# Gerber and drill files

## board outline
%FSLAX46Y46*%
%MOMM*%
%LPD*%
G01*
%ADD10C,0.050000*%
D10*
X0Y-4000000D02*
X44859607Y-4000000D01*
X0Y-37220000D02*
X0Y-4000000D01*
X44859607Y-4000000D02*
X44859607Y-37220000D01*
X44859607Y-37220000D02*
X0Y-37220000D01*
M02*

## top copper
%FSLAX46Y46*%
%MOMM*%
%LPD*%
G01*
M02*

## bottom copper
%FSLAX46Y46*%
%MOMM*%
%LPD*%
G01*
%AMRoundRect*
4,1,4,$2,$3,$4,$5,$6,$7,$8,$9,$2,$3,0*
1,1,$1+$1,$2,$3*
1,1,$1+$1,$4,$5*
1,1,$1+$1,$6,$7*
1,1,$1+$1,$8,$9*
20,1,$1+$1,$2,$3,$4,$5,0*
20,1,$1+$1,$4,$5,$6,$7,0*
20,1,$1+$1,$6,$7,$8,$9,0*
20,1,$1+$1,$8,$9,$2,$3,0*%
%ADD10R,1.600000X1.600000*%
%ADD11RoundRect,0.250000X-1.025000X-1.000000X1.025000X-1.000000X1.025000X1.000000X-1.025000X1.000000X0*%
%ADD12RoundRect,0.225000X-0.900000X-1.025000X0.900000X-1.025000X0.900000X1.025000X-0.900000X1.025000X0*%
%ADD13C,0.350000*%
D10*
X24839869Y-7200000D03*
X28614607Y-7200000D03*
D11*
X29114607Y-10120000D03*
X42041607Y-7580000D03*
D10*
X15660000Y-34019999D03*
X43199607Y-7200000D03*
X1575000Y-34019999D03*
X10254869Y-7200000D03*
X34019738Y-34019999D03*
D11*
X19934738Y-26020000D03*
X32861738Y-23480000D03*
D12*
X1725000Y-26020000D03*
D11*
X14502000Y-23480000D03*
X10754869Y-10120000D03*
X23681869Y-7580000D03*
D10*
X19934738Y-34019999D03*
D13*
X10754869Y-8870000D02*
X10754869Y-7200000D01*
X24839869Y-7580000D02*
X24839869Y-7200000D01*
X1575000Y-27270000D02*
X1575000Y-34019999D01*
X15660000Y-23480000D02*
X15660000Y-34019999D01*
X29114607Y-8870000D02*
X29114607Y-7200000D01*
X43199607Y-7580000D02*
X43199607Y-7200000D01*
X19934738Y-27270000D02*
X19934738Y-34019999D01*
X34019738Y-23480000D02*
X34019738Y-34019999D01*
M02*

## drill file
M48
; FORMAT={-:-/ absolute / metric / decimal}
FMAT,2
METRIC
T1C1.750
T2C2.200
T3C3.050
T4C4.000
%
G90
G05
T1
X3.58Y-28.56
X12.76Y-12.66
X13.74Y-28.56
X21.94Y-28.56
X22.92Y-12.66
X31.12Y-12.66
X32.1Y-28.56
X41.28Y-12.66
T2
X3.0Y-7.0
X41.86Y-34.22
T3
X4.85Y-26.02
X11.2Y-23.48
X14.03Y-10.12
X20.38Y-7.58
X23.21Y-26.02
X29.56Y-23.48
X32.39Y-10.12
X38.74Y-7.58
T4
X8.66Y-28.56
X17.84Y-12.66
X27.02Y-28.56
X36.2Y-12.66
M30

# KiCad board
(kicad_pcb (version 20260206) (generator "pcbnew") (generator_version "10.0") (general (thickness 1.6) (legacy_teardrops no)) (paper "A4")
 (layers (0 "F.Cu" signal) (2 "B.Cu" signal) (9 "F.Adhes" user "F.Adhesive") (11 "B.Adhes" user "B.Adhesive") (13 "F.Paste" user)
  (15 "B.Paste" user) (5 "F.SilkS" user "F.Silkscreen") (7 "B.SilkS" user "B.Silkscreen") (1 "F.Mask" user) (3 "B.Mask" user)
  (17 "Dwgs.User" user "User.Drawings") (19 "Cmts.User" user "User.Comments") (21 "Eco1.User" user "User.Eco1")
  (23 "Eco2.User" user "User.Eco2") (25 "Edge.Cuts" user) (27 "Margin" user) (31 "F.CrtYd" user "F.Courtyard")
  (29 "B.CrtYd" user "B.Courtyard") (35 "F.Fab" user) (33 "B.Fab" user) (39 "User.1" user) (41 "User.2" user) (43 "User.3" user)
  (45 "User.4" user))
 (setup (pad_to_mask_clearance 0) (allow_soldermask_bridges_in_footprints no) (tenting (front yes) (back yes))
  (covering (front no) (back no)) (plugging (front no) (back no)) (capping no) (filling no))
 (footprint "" (layer "F.Cu") (at 0 0)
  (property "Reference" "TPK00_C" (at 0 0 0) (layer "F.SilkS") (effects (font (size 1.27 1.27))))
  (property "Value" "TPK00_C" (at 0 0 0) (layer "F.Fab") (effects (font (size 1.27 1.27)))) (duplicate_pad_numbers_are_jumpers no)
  (pad "1" smd rect (at 24.839869 7.2) (size 1.6 1.6) (layers "B.Cu" "B.Mask") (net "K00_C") (thermal_bridge_angle 45)))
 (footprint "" (layer "F.Cu") (at 0 0)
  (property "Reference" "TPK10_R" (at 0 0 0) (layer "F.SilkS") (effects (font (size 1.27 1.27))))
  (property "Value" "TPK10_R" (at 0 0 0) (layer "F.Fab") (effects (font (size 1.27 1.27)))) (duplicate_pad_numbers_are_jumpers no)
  (pad "1" smd rect (at 28.614607 7.2) (size 1.6 1.6) (layers "B.Cu" "B.Mask") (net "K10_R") (thermal_bridge_angle 45)))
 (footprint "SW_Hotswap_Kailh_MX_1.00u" (layer "F.Cu") (at 36.199607 12.66)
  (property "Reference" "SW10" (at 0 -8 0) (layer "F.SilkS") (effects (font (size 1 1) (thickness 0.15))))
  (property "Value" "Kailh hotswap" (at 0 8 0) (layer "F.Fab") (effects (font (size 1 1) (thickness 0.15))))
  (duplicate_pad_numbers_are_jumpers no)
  (pad "" np_thru_hole circle (at -5.08 0) (size 1.75 1.75) (drill 1.75) (layers "*.Cu" "*.Mask"))
  (pad "" np_thru_hole circle (at -3.81 -2.54) (size 3.05 3.05) (drill 3.05) (layers "*.Cu" "*.Mask"))
  (pad "" np_thru_hole circle (at 0 0) (size 4 4) (drill 4) (layers "*.Cu" "*.Mask"))
  (pad "" np_thru_hole circle (at 2.54 -5.08) (size 3.05 3.05) (drill 3.05) (layers "*.Cu" "*.Mask"))
  (pad "" np_thru_hole circle (at 5.08 0) (size 1.75 1.75) (drill 1.75) (layers "*.Cu" "*.Mask"))
  (pad "1" smd roundrect (at -7.085 -2.54) (size 2.55 2.5) (layers "B.Cu" "B.Mask" "B.Paste") (roundrect_rratio 0.1) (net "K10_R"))
  (pad "2" smd roundrect (at 5.842 -5.08) (size 2.55 2.5) (layers "B.Cu" "B.Mask" "B.Paste") (roundrect_rratio 0.1) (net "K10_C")))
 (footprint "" (layer "F.Cu") (at 0 0)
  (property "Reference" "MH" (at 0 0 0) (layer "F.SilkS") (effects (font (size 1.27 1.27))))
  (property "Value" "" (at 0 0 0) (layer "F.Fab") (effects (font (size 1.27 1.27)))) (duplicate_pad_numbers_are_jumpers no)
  (pad "" np_thru_hole circle (at 41.859607 34.22) (size 2.2 2.2) (drill 2.2) (layers "*.Cu")))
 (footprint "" (layer "F.Cu") (at 0 0)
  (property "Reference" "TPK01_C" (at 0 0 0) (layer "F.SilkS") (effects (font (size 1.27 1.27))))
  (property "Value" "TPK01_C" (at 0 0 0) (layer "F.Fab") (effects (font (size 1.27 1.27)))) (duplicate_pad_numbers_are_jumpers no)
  (pad "1" smd rect (at 15.66 34.019999) (size 1.6 1.6) (layers "B.Cu" "B.Mask") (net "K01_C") (thermal_bridge_angle 45)))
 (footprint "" (layer "F.Cu") (at 0 0)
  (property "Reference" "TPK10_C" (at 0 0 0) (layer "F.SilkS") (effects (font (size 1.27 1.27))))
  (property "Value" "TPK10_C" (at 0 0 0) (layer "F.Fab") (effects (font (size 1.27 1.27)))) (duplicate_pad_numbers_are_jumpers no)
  (pad "1" smd rect (at 43.199607 7.2) (size 1.6 1.6) (layers "B.Cu" "B.Mask") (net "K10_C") (thermal_bridge_angle 45)))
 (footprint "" (layer "F.Cu") (at 0 0)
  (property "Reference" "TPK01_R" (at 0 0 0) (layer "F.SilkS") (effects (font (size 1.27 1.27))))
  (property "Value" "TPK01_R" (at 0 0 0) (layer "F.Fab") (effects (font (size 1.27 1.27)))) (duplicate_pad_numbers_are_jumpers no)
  (pad "1" smd rect (at 1.575 34.019999) (size 1.6 1.6) (layers "B.Cu" "B.Mask") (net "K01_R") (thermal_bridge_angle 45)))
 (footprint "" (layer "F.Cu") (at 0 0)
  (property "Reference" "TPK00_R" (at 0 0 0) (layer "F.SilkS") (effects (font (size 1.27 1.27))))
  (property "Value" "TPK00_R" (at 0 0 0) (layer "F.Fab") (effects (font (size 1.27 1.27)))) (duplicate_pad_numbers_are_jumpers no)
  (pad "1" smd rect (at 10.254869 7.2) (size 1.6 1.6) (layers "B.Cu" "B.Mask") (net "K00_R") (thermal_bridge_angle 45)))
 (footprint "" (layer "F.Cu") (at 0 0)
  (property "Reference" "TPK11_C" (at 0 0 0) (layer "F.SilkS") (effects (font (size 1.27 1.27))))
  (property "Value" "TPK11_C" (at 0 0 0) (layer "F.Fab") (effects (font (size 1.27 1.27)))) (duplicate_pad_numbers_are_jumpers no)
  (pad "1" smd rect (at 34.019738 34.019999) (size 1.6 1.6) (layers "B.Cu" "B.Mask") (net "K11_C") (thermal_bridge_angle 45)))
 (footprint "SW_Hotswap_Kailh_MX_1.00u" (layer "F.Cu") (at 27.019738 28.56)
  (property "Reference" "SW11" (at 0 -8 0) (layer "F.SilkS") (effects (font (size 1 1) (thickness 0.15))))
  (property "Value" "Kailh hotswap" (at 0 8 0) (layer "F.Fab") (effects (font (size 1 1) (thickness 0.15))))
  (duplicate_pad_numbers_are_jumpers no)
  (pad "" np_thru_hole circle (at -5.08 0) (size 1.75 1.75) (drill 1.75) (layers "*.Cu" "*.Mask"))
  (pad "" np_thru_hole circle (at -3.81 -2.54) (size 3.05 3.05) (drill 3.05) (layers "*.Cu" "*.Mask"))
  (pad "" np_thru_hole circle (at 0 0) (size 4 4) (drill 4) (layers "*.Cu" "*.Mask"))
  (pad "" np_thru_hole circle (at 2.54 -5.08) (size 3.05 3.05) (drill 3.05) (layers "*.Cu" "*.Mask"))
  (pad "" np_thru_hole circle (at 5.08 0) (size 1.75 1.75) (drill 1.75) (layers "*.Cu" "*.Mask"))
  (pad "1" smd roundrect (at -7.085 -2.54) (size 2.55 2.5) (layers "B.Cu" "B.Mask" "B.Paste") (roundrect_rratio 0.1) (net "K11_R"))
  (pad "2" smd roundrect (at 5.842 -5.08) (size 2.55 2.5) (layers "B.Cu" "B.Mask" "B.Paste") (roundrect_rratio 0.1) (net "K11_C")))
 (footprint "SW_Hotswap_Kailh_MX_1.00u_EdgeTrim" (layer "F.Cu") (at 8.66 28.56)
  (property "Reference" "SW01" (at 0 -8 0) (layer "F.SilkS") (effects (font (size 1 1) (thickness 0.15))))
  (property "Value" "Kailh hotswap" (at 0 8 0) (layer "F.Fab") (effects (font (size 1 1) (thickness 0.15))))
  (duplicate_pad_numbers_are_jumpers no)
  (pad "" np_thru_hole circle (at -5.08 0) (size 1.75 1.75) (drill 1.75) (layers "*.Cu" "*.Mask"))
  (pad "" np_thru_hole circle (at -3.81 -2.54) (size 3.05 3.05) (drill 3.05) (layers "*.Cu" "*.Mask"))
  (pad "" np_thru_hole circle (at 0 0) (size 4 4) (drill 4) (layers "*.Cu" "*.Mask"))
  (pad "" np_thru_hole circle (at 2.54 -5.08) (size 3.05 3.05) (drill 3.05) (layers "*.Cu" "*.Mask"))
  (pad "" np_thru_hole circle (at 5.08 0) (size 1.75 1.75) (drill 1.75) (layers "*.Cu" "*.Mask"))
  (pad "1" smd roundrect (at -6.935 -2.54) (size 2.25 2.5) (layers "B.Cu" "B.Mask" "B.Paste") (roundrect_rratio 0.1) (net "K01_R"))
  (pad "2" smd roundrect (at 5.842 -5.08) (size 2.55 2.5) (layers "B.Cu" "B.Mask" "B.Paste") (roundrect_rratio 0.1) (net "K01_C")))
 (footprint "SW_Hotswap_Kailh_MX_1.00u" (layer "F.Cu") (at 17.839869 12.66)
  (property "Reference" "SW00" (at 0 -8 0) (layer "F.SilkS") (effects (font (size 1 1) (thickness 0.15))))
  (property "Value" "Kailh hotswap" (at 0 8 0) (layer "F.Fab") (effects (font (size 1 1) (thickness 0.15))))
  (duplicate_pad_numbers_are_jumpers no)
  (pad "" np_thru_hole circle (at -5.08 0) (size 1.75 1.75) (drill 1.75) (layers "*.Cu" "*.Mask"))
  (pad "" np_thru_hole circle (at -3.81 -2.54) (size 3.05 3.05) (drill 3.05) (layers "*.Cu" "*.Mask"))
  (pad "" np_thru_hole circle (at 0 0) (size 4 4) (drill 4) (layers "*.Cu" "*.Mask"))
  (pad "" np_thru_hole circle (at 2.54 -5.08) (size 3.05 3.05) (drill 3.05) (layers "*.Cu" "*.Mask"))
  (pad "" np_thru_hole circle (at 5.08 0) (size 1.75 1.75) (drill 1.75) (layers "*.Cu" "*.Mask"))
  (pad "1" smd roundrect (at -7.085 -2.54) (size 2.55 2.5) (layers "B.Cu" "B.Mask" "B.Paste") (roundrect_rratio 0.1) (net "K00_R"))
  (pad "2" smd roundrect (at 5.842 -5.08) (size 2.55 2.5) (layers "B.Cu" "B.Mask" "B.Paste") (roundrect_rratio 0.1) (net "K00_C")))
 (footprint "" (layer "F.Cu") (at 0 0)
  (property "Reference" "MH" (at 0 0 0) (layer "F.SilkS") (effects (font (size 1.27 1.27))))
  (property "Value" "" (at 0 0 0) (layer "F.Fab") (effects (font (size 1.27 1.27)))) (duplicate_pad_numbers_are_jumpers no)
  (pad "" np_thru_hole circle (at 3 7) (size 2.2 2.2) (drill 2.2) (layers "*.Cu")))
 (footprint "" (layer "F.Cu") (at 0 0)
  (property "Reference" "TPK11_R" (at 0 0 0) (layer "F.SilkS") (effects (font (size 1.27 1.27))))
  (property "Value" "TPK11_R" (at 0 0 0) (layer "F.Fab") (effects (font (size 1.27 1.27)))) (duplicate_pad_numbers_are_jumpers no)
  (pad "1" smd rect (at 19.934738 34.019999) (size 1.6 1.6) (layers "B.Cu" "B.Mask") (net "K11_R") (thermal_bridge_angle 45)))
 (gr_line (start 0 4) (end 44.859607 4) (stroke (width 0.05) (type default)) (layer "Edge.Cuts"))
 (gr_line (start 0 37.22) (end 0 4) (stroke (width 0.05) (type default)) (layer "Edge.Cuts"))
 (gr_line (start 44.859607 4) (end 44.859607 37.22) (stroke (width 0.05) (type default)) (layer "Edge.Cuts"))
 (gr_line (start 44.859607 37.22) (end 0 37.22) (stroke (width 0.05) (type default)) (layer "Edge.Cuts"))
 (segment (start 10.754869 8.87) (end 10.754869 7.2) (width 0.35) (layer "B.Cu") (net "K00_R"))
 (segment (start 24.839869 7.58) (end 24.839869 7.2) (width 0.35) (layer "B.Cu") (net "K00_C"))
 (segment (start 1.575 27.27) (end 1.575 34.019999) (width 0.35) (layer "B.Cu") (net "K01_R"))
 (segment (start 15.66 23.48) (end 15.66 34.019999) (width 0.35) (layer "B.Cu") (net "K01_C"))
 (segment (start 29.114607 8.87) (end 29.114607 7.2) (width 0.35) (layer "B.Cu") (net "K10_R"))
 (segment (start 43.199607 7.58) (end 43.199607 7.2) (width 0.35) (layer "B.Cu") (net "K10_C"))
 (segment (start 19.934738 27.27) (end 19.934738 34.019999) (width 0.35) (layer "B.Cu") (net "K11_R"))
 (segment (start 34.019738 23.48) (end 34.019738 34.019999) (width 0.35) (layer "B.Cu") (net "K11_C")))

